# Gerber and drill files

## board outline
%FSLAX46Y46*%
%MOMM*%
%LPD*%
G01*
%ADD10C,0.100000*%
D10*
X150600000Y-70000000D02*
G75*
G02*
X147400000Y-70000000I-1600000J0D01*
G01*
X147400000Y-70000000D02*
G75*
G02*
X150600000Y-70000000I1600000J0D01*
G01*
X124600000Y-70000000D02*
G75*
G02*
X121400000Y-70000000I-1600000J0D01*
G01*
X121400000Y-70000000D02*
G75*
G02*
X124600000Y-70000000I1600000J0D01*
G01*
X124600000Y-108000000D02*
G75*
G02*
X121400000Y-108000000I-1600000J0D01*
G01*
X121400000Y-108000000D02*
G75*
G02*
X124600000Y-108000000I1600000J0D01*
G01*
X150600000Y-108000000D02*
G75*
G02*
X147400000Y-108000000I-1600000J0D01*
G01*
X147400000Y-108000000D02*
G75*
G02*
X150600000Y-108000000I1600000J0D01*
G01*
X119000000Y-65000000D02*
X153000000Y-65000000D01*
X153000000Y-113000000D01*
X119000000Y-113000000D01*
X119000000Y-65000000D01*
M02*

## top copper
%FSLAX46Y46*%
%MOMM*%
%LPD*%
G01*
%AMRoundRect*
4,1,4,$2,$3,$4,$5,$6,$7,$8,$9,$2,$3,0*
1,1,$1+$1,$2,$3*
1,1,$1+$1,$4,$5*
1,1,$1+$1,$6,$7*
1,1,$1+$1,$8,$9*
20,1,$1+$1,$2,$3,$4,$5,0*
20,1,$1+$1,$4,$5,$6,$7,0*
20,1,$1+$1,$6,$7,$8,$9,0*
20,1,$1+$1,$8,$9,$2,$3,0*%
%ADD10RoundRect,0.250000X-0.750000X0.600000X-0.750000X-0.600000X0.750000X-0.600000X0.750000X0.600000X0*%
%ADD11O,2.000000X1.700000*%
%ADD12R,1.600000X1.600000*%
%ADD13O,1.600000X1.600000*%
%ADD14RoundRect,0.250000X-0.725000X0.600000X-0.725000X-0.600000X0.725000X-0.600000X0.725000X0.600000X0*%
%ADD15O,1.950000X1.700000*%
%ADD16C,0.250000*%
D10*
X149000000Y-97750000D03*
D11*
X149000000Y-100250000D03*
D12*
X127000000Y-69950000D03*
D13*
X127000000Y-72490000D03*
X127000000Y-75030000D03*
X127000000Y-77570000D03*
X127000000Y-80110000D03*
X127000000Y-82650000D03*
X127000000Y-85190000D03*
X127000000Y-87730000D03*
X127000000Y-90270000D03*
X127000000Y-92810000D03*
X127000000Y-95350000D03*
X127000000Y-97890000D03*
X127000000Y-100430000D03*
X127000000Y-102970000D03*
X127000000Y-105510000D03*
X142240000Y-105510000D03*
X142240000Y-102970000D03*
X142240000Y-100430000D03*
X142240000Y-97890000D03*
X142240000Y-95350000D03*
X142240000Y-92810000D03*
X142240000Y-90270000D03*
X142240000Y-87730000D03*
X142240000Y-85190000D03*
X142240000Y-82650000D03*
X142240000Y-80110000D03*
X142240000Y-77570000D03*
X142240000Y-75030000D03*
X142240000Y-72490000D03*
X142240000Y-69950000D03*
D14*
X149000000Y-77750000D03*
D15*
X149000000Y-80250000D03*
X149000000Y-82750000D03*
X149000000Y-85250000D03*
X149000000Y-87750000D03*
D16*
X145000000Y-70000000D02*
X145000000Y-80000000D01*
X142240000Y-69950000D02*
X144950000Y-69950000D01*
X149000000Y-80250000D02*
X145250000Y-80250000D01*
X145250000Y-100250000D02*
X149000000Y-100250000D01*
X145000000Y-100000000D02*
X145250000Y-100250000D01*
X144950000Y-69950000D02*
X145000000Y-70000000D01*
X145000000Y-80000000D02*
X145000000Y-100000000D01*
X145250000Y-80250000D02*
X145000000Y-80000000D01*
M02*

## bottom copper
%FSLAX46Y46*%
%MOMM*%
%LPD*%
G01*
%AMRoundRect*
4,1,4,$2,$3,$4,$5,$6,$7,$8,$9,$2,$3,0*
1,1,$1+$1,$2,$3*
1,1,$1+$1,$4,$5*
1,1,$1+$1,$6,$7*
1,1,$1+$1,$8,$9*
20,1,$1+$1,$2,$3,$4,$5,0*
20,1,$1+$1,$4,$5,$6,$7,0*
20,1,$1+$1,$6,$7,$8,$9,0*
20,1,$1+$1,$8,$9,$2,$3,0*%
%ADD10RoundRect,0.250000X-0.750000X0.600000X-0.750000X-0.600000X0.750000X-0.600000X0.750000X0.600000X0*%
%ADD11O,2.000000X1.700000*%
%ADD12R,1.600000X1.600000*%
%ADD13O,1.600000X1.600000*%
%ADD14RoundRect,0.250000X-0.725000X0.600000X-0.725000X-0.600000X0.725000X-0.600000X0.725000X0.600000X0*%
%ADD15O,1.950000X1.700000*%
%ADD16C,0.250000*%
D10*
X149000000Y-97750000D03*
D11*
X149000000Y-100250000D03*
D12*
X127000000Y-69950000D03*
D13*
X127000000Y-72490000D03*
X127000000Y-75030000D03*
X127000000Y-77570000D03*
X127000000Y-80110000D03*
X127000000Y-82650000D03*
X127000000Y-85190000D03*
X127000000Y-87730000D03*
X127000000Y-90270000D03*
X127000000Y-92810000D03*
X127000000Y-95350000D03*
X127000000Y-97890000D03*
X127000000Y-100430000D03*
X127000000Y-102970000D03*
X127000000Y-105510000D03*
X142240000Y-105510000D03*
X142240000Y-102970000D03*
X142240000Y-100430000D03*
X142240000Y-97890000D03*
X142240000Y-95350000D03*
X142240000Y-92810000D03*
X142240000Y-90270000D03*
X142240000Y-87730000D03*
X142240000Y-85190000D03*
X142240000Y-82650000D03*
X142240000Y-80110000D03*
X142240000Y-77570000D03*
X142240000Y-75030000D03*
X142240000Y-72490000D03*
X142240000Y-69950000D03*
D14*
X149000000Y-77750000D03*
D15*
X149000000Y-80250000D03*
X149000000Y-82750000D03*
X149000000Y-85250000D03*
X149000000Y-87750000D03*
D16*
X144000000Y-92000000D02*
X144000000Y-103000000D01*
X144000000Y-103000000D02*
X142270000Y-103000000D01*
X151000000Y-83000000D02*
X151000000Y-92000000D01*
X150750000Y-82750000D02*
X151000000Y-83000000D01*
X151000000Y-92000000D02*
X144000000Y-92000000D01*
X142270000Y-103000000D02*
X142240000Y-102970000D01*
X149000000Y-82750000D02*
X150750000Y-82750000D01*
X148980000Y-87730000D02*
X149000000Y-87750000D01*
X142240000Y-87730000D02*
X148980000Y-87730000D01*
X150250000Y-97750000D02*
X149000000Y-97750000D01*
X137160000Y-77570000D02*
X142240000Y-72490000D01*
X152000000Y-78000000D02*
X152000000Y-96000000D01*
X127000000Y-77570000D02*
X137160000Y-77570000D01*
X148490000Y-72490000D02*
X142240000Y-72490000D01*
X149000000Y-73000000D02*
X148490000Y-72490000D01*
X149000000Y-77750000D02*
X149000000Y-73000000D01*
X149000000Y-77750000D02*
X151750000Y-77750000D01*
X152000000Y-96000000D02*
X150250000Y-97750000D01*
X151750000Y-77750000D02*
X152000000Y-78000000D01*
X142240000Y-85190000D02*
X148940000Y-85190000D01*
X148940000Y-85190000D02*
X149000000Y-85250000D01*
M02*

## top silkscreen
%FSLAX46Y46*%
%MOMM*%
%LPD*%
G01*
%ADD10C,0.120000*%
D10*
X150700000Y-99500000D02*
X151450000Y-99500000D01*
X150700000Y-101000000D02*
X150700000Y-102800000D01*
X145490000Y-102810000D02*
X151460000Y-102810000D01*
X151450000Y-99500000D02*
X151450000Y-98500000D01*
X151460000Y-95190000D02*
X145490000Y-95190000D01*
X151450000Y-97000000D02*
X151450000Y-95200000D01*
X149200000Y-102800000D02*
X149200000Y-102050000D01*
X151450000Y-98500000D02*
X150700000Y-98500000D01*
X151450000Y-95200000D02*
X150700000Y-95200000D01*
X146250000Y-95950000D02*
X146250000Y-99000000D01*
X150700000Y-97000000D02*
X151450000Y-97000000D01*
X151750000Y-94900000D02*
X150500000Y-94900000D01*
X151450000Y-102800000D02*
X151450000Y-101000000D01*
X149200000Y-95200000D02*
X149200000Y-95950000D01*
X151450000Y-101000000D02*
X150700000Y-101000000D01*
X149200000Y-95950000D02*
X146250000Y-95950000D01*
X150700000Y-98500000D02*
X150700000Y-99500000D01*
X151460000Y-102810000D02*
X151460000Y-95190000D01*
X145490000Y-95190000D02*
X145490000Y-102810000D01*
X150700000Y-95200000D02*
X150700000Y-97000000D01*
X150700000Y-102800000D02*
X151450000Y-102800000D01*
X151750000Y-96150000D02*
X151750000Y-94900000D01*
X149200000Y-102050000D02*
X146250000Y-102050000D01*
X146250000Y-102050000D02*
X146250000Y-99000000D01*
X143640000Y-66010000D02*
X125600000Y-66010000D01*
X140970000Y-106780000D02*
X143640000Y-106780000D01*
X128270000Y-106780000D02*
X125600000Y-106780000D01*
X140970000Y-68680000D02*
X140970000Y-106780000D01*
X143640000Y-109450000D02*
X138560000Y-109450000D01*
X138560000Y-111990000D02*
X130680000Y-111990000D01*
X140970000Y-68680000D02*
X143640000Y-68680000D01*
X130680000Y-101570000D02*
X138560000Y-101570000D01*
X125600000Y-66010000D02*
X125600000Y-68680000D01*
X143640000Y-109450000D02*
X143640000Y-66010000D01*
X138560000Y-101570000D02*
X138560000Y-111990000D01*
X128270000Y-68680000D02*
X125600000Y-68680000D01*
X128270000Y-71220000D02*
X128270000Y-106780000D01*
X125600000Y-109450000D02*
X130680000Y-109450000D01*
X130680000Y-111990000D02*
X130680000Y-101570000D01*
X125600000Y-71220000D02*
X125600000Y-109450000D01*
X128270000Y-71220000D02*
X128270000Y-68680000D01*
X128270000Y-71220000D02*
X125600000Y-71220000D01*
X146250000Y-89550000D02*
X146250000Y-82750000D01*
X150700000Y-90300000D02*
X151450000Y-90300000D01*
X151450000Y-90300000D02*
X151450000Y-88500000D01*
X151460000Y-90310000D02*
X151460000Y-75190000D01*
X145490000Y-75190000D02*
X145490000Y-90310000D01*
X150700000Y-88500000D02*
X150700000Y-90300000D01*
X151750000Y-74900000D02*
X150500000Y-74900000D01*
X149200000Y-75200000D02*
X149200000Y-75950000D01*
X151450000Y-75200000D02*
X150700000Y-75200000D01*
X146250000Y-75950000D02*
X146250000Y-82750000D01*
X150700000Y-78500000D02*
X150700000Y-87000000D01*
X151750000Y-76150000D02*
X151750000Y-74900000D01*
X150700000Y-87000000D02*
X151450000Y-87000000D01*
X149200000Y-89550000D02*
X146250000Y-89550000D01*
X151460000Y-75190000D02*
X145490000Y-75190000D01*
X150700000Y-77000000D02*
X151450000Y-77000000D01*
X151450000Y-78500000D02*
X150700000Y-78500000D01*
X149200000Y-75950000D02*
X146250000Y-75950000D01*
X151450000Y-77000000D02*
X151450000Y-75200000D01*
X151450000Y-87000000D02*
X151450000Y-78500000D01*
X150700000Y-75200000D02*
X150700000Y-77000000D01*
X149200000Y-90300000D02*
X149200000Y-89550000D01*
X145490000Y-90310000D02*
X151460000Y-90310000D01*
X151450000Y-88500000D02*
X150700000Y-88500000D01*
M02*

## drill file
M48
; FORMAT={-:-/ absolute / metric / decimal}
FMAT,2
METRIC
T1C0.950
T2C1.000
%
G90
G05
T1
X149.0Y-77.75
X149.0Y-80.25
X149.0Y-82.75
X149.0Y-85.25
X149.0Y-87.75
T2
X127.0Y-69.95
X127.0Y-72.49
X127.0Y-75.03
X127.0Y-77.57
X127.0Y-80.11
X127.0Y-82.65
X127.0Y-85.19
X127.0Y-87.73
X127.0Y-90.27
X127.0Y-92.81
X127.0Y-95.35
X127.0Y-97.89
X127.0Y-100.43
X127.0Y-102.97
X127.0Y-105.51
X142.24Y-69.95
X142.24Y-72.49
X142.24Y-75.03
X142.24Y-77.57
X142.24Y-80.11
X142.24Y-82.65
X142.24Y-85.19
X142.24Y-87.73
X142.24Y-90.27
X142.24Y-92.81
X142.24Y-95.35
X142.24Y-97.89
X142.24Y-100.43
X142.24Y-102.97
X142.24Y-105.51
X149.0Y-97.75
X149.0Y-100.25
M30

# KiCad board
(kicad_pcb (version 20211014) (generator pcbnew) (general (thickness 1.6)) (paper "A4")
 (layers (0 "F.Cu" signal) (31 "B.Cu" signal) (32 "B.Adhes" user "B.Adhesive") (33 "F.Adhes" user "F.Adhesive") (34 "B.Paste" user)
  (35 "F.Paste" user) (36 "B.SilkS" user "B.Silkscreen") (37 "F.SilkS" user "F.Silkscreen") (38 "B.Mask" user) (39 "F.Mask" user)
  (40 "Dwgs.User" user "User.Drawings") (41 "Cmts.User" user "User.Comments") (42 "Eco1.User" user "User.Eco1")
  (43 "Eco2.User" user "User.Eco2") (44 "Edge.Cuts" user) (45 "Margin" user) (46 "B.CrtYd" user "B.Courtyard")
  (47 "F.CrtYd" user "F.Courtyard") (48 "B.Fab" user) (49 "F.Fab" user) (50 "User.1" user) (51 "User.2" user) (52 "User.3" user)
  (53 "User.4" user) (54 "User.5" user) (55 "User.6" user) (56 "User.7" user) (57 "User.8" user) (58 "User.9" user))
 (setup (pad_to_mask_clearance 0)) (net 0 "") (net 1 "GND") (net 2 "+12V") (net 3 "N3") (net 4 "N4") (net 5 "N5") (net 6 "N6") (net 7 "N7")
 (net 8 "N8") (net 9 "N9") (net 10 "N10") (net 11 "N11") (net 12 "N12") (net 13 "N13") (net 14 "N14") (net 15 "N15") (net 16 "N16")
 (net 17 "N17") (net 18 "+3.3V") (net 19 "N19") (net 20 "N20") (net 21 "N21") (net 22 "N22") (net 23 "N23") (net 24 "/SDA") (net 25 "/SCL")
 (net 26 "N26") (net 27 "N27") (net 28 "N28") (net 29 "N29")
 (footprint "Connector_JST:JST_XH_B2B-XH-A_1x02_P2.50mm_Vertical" (layer "F.Cu") (at 149 97.75 -90)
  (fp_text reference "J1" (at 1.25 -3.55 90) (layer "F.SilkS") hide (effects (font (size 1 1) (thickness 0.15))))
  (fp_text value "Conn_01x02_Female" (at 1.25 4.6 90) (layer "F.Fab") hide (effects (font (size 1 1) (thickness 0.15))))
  (fp_line (start 1.75 -1.7) (end 1.75 -2.45) (layer "F.SilkS") (width 0.12))
  (fp_line (start 3.25 -1.7) (end 5.05 -1.7) (layer "F.SilkS") (width 0.12))
  (fp_line (start 5.06 3.51) (end 5.06 -2.46) (layer "F.SilkS") (width 0.12))
  (fp_line (start 1.75 -2.45) (end 0.75 -2.45) (layer "F.SilkS") (width 0.12))
  (fp_line (start -2.56 -2.46) (end -2.56 3.51) (layer "F.SilkS") (width 0.12))
  (fp_line (start -0.75 -2.45) (end -2.55 -2.45) (layer "F.SilkS") (width 0.12))
  (fp_line (start 5.05 -0.2) (end 4.3 -0.2) (layer "F.SilkS") (width 0.12))
  (fp_line (start 0.75 -2.45) (end 0.75 -1.7) (layer "F.SilkS") (width 0.12))
  (fp_line (start -2.55 -2.45) (end -2.55 -1.7) (layer "F.SilkS") (width 0.12))
  (fp_line (start -1.8 2.75) (end 1.25 2.75) (layer "F.SilkS") (width 0.12))
  (fp_line (start -0.75 -1.7) (end -0.75 -2.45) (layer "F.SilkS") (width 0.12))
  (fp_line (start -2.85 -2.75) (end -2.85 -1.5) (layer "F.SilkS") (width 0.12))
  (fp_line (start 5.05 -2.45) (end 3.25 -2.45) (layer "F.SilkS") (width 0.12))
  (fp_line (start -2.55 -0.2) (end -1.8 -0.2) (layer "F.SilkS") (width 0.12))
  (fp_line (start 3.25 -2.45) (end 3.25 -1.7) (layer "F.SilkS") (width 0.12))
  (fp_line (start -1.8 -0.2) (end -1.8 2.75) (layer "F.SilkS") (width 0.12))
  (fp_line (start 0.75 -1.7) (end 1.75 -1.7) (layer "F.SilkS") (width 0.12))
  (fp_line (start 5.06 -2.46) (end -2.56 -2.46) (layer "F.SilkS") (width 0.12))
  (fp_line (start -2.56 3.51) (end 5.06 3.51) (layer "F.SilkS") (width 0.12))
  (fp_line (start -2.55 -1.7) (end -0.75 -1.7) (layer "F.SilkS") (width 0.12))
  (fp_line (start 5.05 -1.7) (end 5.05 -2.45) (layer "F.SilkS") (width 0.12))
  (fp_line (start -1.6 -2.75) (end -2.85 -2.75) (layer "F.SilkS") (width 0.12))
  (fp_line (start 4.3 -0.2) (end 4.3 2.75) (layer "F.SilkS") (width 0.12))
  (fp_line (start 4.3 2.75) (end 1.25 2.75) (layer "F.SilkS") (width 0.12))
  (pad "1" thru_hole roundrect (at 0 0 270) (size 1.7 2) (drill 1) (layers *.Cu *.Mask) (roundrect_rratio 0.1470588235) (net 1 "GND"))
  (pad "2" thru_hole oval (at 2.5 0 270) (size 1.7 2) (drill 1) (layers *.Cu *.Mask) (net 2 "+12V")))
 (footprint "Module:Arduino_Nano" (layer "F.Cu") (at 127 69.95)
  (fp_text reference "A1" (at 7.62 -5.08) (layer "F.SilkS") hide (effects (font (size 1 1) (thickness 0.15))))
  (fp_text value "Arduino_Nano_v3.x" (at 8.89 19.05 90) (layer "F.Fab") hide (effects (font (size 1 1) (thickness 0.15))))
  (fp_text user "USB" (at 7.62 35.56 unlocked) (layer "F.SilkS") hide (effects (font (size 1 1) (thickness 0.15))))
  (fp_line (start 16.64 -3.94) (end -1.4 -3.94) (layer "F.SilkS") (width 0.12))
  (fp_line (start 13.97 36.83) (end 16.64 36.83) (layer "F.SilkS") (width 0.12))
  (fp_line (start 1.27 36.83) (end -1.4 36.83) (layer "F.SilkS") (width 0.12))
  (fp_line (start 13.97 -1.27) (end 13.97 36.83) (layer "F.SilkS") (width 0.12))
  (fp_line (start 16.64 39.5) (end 11.56 39.5) (layer "F.SilkS") (width 0.12))
  (fp_line (start 11.56 42.04) (end 3.68 42.04) (layer "F.SilkS") (width 0.12))
  (fp_line (start 13.97 -1.27) (end 16.64 -1.27) (layer "F.SilkS") (width 0.12))
  (fp_line (start 3.68 31.62) (end 11.56 31.62) (layer "F.SilkS") (width 0.12))
  (fp_line (start -1.4 -3.94) (end -1.4 -1.27) (layer "F.SilkS") (width 0.12))
  (fp_line (start 16.64 39.5) (end 16.64 -3.94) (layer "F.SilkS") (width 0.12))
  (fp_line (start 11.56 31.62) (end 11.56 42.04) (layer "F.SilkS") (width 0.12))
  (fp_line (start 1.27 -1.27) (end -1.4 -1.27) (layer "F.SilkS") (width 0.12))
  (fp_line (start 1.27 1.27) (end 1.27 36.83) (layer "F.SilkS") (width 0.12))
  (fp_line (start -1.4 39.5) (end 3.68 39.5) (layer "F.SilkS") (width 0.12))
  (fp_line (start 3.68 42.04) (end 3.68 31.62) (layer "F.SilkS") (width 0.12))
  (fp_line (start -1.4 1.27) (end -1.4 39.5) (layer "F.SilkS") (width 0.12))
  (fp_line (start 1.27 1.27) (end 1.27 -1.27) (layer "F.SilkS") (width 0.12))
  (fp_line (start 1.27 1.27) (end -1.4 1.27) (layer "F.SilkS") (width 0.12))
  (pad "1" thru_hole rect (at 0 0) (size 1.6 1.6) (drill 1) (layers *.Cu *.Mask) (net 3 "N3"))
  (pad "2" thru_hole oval (at 0 2.54) (size 1.6 1.6) (drill 1) (layers *.Cu *.Mask) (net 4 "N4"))
  (pad "3" thru_hole oval (at 0 5.08) (size 1.6 1.6) (drill 1) (layers *.Cu *.Mask) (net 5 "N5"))
  (pad "4" thru_hole oval (at 0 7.62) (size 1.6 1.6) (drill 1) (layers *.Cu *.Mask) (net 1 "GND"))
  (pad "5" thru_hole oval (at 0 10.16) (size 1.6 1.6) (drill 1) (layers *.Cu *.Mask) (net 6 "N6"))
  (pad "6" thru_hole oval (at 0 12.7) (size 1.6 1.6) (drill 1) (layers *.Cu *.Mask) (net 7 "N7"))
  (pad "7" thru_hole oval (at 0 15.24) (size 1.6 1.6) (drill 1) (layers *.Cu *.Mask) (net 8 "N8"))
  (pad "8" thru_hole oval (at 0 17.78) (size 1.6 1.6) (drill 1) (layers *.Cu *.Mask) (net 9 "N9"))
  (pad "9" thru_hole oval (at 0 20.32) (size 1.6 1.6) (drill 1) (layers *.Cu *.Mask) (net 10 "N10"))
  (pad "10" thru_hole oval (at 0 22.86) (size 1.6 1.6) (drill 1) (layers *.Cu *.Mask) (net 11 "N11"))
  (pad "11" thru_hole oval (at 0 25.4) (size 1.6 1.6) (drill 1) (layers *.Cu *.Mask) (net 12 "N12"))
  (pad "12" thru_hole oval (at 0 27.94) (size 1.6 1.6) (drill 1) (layers *.Cu *.Mask) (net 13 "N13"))
  (pad "13" thru_hole oval (at 0 30.48) (size 1.6 1.6) (drill 1) (layers *.Cu *.Mask) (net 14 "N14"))
  (pad "14" thru_hole oval (at 0 33.02) (size 1.6 1.6) (drill 1) (layers *.Cu *.Mask) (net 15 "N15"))
  (pad "15" thru_hole oval (at 0 35.56) (size 1.6 1.6) (drill 1) (layers *.Cu *.Mask) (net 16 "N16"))
  (pad "16" thru_hole oval (at 15.24 35.56) (size 1.6 1.6) (drill 1) (layers *.Cu *.Mask) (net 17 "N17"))
  (pad "17" thru_hole oval (at 15.24 33.02) (size 1.6 1.6) (drill 1) (layers *.Cu *.Mask) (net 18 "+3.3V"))
  (pad "18" thru_hole oval (at 15.24 30.48) (size 1.6 1.6) (drill 1) (layers *.Cu *.Mask) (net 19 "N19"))
  (pad "19" thru_hole oval (at 15.24 27.94) (size 1.6 1.6) (drill 1) (layers *.Cu *.Mask) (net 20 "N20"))
  (pad "20" thru_hole oval (at 15.24 25.4) (size 1.6 1.6) (drill 1) (layers *.Cu *.Mask) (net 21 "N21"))
  (pad "21" thru_hole oval (at 15.24 22.86) (size 1.6 1.6) (drill 1) (layers *.Cu *.Mask) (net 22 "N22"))
  (pad "22" thru_hole oval (at 15.24 20.32) (size 1.6 1.6) (drill 1) (layers *.Cu *.Mask) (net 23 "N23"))
  (pad "23" thru_hole oval (at 15.24 17.78) (size 1.6 1.6) (drill 1) (layers *.Cu *.Mask) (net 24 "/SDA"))
  (pad "24" thru_hole oval (at 15.24 15.24) (size 1.6 1.6) (drill 1) (layers *.Cu *.Mask) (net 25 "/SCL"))
  (pad "25" thru_hole oval (at 15.24 12.7) (size 1.6 1.6) (drill 1) (layers *.Cu *.Mask) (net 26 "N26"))
  (pad "26" thru_hole oval (at 15.24 10.16) (size 1.6 1.6) (drill 1) (layers *.Cu *.Mask) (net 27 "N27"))
  (pad "27" thru_hole oval (at 15.24 7.62) (size 1.6 1.6) (drill 1) (layers *.Cu *.Mask) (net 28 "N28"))
  (pad "28" thru_hole oval (at 15.24 5.08) (size 1.6 1.6) (drill 1) (layers *.Cu *.Mask) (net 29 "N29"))
  (pad "29" thru_hole oval (at 15.24 2.54) (size 1.6 1.6) (drill 1) (layers *.Cu *.Mask) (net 1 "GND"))
  (pad "30" thru_hole oval (at 15.24 0) (size 1.6 1.6) (drill 1) (layers *.Cu *.Mask) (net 2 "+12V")))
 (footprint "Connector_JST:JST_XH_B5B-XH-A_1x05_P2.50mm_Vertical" (layer "F.Cu") (at 149 77.75 -90)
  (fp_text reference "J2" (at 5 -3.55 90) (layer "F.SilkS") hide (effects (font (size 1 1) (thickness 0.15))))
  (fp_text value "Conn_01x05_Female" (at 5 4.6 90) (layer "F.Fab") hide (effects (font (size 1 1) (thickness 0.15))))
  (fp_line (start 11.8 2.75) (end 5 2.75) (layer "F.SilkS") (width 0.12))
  (fp_line (start 12.55 -1.7) (end 12.55 -2.45) (layer "F.SilkS") (width 0.12))
  (fp_line (start 12.55 -2.45) (end 10.75 -2.45) (layer "F.SilkS") (width 0.12))
  (fp_line (start 12.56 -2.46) (end -2.56 -2.46) (layer "F.SilkS") (width 0.12))
  (fp_line (start -2.56 3.51) (end 12.56 3.51) (layer "F.SilkS") (width 0.12))
  (fp_line (start 10.75 -1.7) (end 12.55 -1.7) (layer "F.SilkS") (width 0.12))
  (fp_line (start -2.85 -2.75) (end -2.85 -1.5) (layer "F.SilkS") (width 0.12))
  (fp_line (start -2.55 -0.2) (end -1.8 -0.2) (layer "F.SilkS") (width 0.12))
  (fp_line (start -2.55 -2.45) (end -2.55 -1.7) (layer "F.SilkS") (width 0.12))
  (fp_line (start -1.8 2.75) (end 5 2.75) (layer "F.SilkS") (width 0.12))
  (fp_line (start 0.75 -1.7) (end 9.25 -1.7) (layer "F.SilkS") (width 0.12))
  (fp_line (start -1.6 -2.75) (end -2.85 -2.75) (layer "F.SilkS") (width 0.12))
  (fp_line (start 9.25 -1.7) (end 9.25 -2.45) (layer "F.SilkS") (width 0.12))
  (fp_line (start 11.8 -0.2) (end 11.8 2.75) (layer "F.SilkS") (width 0.12))
  (fp_line (start -2.56 -2.46) (end -2.56 3.51) (layer "F.SilkS") (width 0.12))
  (fp_line (start -0.75 -1.7) (end -0.75 -2.45) (layer "F.SilkS") (width 0.12))
  (fp_line (start 0.75 -2.45) (end 0.75 -1.7) (layer "F.SilkS") (width 0.12))
  (fp_line (start -1.8 -0.2) (end -1.8 2.75) (layer "F.SilkS") (width 0.12))
  (fp_line (start -0.75 -2.45) (end -2.55 -2.45) (layer "F.SilkS") (width 0.12))
  (fp_line (start 9.25 -2.45) (end 0.75 -2.45) (layer "F.SilkS") (width 0.12))
  (fp_line (start -2.55 -1.7) (end -0.75 -1.7) (layer "F.SilkS") (width 0.12))
  (fp_line (start 12.55 -0.2) (end 11.8 -0.2) (layer "F.SilkS") (width 0.12))
  (fp_line (start 12.56 3.51) (end 12.56 -2.46) (layer "F.SilkS") (width 0.12))
  (fp_line (start 10.75 -2.45) (end 10.75 -1.7) (layer "F.SilkS") (width 0.12))
  (pad "1" thru_hole roundrect (at 0 0 270) (size 1.7 1.95) (drill 0.95) (layers *.Cu *.Mask) (roundrect_rratio 0.1470588235) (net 1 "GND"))
  (pad "2" thru_hole oval (at 2.5 0 270) (size 1.7 1.95) (drill 0.95) (layers *.Cu *.Mask) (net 2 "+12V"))
  (pad "3" thru_hole oval (at 5 0 270) (size 1.7 1.95) (drill 0.95) (layers *.Cu *.Mask) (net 18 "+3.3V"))
  (pad "4" thru_hole oval (at 7.5 0 270) (size 1.7 1.95) (drill 0.95) (layers *.Cu *.Mask) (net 25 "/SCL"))
  (pad "5" thru_hole oval (at 10 0 270) (size 1.7 1.95) (drill 0.95) (layers *.Cu *.Mask) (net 24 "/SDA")))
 (gr_circle (center 149 70) (end 150.6 70) (layer "Edge.Cuts") (width 0.1) (fill none))
 (gr_circle (center 123 70) (end 124.6 70) (layer "Edge.Cuts") (width 0.1) (fill none))
 (gr_circle (center 123 108) (end 124.6 108) (layer "Edge.Cuts") (width 0.1) (fill none))
 (gr_circle (center 149 108) (end 150.6 108) (layer "Edge.Cuts") (width 0.1) (fill none))
 (gr_rect (start 153 113) (end 119 65) (layer "Edge.Cuts") (width 0.1) (fill none))
 (segment (start 144 92) (end 144 103) (width 0.25) (layer "B.Cu") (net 18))
 (segment (start 144 103) (end 142.27 103) (width 0.25) (layer "B.Cu") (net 18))
 (segment (start 151 83) (end 151 92) (width 0.25) (layer "B.Cu") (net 18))
 (segment (start 150.75 82.75) (end 151 83) (width 0.25) (layer "B.Cu") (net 18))
 (segment (start 151 92) (end 144 92) (width 0.25) (layer "B.Cu") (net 18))
 (segment (start 142.27 103) (end 142.24 102.97) (width 0.25) (layer "B.Cu") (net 18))
 (segment (start 149 82.75) (end 150.75 82.75) (width 0.25) (layer "B.Cu") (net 18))
 (segment (start 148.98 87.73) (end 149 87.75) (width 0.25) (layer "B.Cu") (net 24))
 (segment (start 142.24 87.73) (end 148.98 87.73) (width 0.25) (layer "B.Cu") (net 24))
 (segment (start 150.25 97.75) (end 149 97.75) (width 0.25) (layer "B.Cu") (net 1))
 (segment (start 137.16 77.57) (end 142.24 72.49) (width 0.25) (layer "B.Cu") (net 1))
 (segment (start 152 78) (end 152 96) (width 0.25) (layer "B.Cu") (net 1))
 (segment (start 127 77.57) (end 137.16 77.57) (width 0.25) (layer "B.Cu") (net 1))
 (segment (start 148.49 72.49) (end 142.24 72.49) (width 0.25) (layer "B.Cu") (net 1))
 (segment (start 149 73) (end 148.49 72.49) (width 0.25) (layer "B.Cu") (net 1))
 (segment (start 149 77.75) (end 149 73) (width 0.25) (layer "B.Cu") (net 1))
 (segment (start 149 77.75) (end 151.75 77.75) (width 0.25) (layer "B.Cu") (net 1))
 (segment (start 152 96) (end 150.25 97.75) (width 0.25) (layer "B.Cu") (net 1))
 (segment (start 151.75 77.75) (end 152 78) (width 0.25) (layer "B.Cu") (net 1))
 (segment (start 145 70) (end 145 80) (width 0.25) (layer "F.Cu") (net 2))
 (segment (start 142.24 69.95) (end 144.95 69.95) (width 0.25) (layer "F.Cu") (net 2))
 (segment (start 149 80.25) (end 145.25 80.25) (width 0.25) (layer "F.Cu") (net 2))
 (segment (start 145.25 100.25) (end 149 100.25) (width 0.25) (layer "F.Cu") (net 2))
 (segment (start 145 100) (end 145.25 100.25) (width 0.25) (layer "F.Cu") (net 2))
 (segment (start 144.95 69.95) (end 145 70) (width 0.25) (layer "F.Cu") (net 2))
 (segment (start 145 80) (end 145 100) (width 0.25) (layer "F.Cu") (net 2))
 (segment (start 145.25 80.25) (end 145 80) (width 0.25) (layer "F.Cu") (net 2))
 (segment (start 142.24 85.19) (end 148.94 85.19) (width 0.25) (layer "B.Cu") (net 25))
 (segment (start 148.94 85.19) (end 149 85.25) (width 0.25) (layer "B.Cu") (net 25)))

